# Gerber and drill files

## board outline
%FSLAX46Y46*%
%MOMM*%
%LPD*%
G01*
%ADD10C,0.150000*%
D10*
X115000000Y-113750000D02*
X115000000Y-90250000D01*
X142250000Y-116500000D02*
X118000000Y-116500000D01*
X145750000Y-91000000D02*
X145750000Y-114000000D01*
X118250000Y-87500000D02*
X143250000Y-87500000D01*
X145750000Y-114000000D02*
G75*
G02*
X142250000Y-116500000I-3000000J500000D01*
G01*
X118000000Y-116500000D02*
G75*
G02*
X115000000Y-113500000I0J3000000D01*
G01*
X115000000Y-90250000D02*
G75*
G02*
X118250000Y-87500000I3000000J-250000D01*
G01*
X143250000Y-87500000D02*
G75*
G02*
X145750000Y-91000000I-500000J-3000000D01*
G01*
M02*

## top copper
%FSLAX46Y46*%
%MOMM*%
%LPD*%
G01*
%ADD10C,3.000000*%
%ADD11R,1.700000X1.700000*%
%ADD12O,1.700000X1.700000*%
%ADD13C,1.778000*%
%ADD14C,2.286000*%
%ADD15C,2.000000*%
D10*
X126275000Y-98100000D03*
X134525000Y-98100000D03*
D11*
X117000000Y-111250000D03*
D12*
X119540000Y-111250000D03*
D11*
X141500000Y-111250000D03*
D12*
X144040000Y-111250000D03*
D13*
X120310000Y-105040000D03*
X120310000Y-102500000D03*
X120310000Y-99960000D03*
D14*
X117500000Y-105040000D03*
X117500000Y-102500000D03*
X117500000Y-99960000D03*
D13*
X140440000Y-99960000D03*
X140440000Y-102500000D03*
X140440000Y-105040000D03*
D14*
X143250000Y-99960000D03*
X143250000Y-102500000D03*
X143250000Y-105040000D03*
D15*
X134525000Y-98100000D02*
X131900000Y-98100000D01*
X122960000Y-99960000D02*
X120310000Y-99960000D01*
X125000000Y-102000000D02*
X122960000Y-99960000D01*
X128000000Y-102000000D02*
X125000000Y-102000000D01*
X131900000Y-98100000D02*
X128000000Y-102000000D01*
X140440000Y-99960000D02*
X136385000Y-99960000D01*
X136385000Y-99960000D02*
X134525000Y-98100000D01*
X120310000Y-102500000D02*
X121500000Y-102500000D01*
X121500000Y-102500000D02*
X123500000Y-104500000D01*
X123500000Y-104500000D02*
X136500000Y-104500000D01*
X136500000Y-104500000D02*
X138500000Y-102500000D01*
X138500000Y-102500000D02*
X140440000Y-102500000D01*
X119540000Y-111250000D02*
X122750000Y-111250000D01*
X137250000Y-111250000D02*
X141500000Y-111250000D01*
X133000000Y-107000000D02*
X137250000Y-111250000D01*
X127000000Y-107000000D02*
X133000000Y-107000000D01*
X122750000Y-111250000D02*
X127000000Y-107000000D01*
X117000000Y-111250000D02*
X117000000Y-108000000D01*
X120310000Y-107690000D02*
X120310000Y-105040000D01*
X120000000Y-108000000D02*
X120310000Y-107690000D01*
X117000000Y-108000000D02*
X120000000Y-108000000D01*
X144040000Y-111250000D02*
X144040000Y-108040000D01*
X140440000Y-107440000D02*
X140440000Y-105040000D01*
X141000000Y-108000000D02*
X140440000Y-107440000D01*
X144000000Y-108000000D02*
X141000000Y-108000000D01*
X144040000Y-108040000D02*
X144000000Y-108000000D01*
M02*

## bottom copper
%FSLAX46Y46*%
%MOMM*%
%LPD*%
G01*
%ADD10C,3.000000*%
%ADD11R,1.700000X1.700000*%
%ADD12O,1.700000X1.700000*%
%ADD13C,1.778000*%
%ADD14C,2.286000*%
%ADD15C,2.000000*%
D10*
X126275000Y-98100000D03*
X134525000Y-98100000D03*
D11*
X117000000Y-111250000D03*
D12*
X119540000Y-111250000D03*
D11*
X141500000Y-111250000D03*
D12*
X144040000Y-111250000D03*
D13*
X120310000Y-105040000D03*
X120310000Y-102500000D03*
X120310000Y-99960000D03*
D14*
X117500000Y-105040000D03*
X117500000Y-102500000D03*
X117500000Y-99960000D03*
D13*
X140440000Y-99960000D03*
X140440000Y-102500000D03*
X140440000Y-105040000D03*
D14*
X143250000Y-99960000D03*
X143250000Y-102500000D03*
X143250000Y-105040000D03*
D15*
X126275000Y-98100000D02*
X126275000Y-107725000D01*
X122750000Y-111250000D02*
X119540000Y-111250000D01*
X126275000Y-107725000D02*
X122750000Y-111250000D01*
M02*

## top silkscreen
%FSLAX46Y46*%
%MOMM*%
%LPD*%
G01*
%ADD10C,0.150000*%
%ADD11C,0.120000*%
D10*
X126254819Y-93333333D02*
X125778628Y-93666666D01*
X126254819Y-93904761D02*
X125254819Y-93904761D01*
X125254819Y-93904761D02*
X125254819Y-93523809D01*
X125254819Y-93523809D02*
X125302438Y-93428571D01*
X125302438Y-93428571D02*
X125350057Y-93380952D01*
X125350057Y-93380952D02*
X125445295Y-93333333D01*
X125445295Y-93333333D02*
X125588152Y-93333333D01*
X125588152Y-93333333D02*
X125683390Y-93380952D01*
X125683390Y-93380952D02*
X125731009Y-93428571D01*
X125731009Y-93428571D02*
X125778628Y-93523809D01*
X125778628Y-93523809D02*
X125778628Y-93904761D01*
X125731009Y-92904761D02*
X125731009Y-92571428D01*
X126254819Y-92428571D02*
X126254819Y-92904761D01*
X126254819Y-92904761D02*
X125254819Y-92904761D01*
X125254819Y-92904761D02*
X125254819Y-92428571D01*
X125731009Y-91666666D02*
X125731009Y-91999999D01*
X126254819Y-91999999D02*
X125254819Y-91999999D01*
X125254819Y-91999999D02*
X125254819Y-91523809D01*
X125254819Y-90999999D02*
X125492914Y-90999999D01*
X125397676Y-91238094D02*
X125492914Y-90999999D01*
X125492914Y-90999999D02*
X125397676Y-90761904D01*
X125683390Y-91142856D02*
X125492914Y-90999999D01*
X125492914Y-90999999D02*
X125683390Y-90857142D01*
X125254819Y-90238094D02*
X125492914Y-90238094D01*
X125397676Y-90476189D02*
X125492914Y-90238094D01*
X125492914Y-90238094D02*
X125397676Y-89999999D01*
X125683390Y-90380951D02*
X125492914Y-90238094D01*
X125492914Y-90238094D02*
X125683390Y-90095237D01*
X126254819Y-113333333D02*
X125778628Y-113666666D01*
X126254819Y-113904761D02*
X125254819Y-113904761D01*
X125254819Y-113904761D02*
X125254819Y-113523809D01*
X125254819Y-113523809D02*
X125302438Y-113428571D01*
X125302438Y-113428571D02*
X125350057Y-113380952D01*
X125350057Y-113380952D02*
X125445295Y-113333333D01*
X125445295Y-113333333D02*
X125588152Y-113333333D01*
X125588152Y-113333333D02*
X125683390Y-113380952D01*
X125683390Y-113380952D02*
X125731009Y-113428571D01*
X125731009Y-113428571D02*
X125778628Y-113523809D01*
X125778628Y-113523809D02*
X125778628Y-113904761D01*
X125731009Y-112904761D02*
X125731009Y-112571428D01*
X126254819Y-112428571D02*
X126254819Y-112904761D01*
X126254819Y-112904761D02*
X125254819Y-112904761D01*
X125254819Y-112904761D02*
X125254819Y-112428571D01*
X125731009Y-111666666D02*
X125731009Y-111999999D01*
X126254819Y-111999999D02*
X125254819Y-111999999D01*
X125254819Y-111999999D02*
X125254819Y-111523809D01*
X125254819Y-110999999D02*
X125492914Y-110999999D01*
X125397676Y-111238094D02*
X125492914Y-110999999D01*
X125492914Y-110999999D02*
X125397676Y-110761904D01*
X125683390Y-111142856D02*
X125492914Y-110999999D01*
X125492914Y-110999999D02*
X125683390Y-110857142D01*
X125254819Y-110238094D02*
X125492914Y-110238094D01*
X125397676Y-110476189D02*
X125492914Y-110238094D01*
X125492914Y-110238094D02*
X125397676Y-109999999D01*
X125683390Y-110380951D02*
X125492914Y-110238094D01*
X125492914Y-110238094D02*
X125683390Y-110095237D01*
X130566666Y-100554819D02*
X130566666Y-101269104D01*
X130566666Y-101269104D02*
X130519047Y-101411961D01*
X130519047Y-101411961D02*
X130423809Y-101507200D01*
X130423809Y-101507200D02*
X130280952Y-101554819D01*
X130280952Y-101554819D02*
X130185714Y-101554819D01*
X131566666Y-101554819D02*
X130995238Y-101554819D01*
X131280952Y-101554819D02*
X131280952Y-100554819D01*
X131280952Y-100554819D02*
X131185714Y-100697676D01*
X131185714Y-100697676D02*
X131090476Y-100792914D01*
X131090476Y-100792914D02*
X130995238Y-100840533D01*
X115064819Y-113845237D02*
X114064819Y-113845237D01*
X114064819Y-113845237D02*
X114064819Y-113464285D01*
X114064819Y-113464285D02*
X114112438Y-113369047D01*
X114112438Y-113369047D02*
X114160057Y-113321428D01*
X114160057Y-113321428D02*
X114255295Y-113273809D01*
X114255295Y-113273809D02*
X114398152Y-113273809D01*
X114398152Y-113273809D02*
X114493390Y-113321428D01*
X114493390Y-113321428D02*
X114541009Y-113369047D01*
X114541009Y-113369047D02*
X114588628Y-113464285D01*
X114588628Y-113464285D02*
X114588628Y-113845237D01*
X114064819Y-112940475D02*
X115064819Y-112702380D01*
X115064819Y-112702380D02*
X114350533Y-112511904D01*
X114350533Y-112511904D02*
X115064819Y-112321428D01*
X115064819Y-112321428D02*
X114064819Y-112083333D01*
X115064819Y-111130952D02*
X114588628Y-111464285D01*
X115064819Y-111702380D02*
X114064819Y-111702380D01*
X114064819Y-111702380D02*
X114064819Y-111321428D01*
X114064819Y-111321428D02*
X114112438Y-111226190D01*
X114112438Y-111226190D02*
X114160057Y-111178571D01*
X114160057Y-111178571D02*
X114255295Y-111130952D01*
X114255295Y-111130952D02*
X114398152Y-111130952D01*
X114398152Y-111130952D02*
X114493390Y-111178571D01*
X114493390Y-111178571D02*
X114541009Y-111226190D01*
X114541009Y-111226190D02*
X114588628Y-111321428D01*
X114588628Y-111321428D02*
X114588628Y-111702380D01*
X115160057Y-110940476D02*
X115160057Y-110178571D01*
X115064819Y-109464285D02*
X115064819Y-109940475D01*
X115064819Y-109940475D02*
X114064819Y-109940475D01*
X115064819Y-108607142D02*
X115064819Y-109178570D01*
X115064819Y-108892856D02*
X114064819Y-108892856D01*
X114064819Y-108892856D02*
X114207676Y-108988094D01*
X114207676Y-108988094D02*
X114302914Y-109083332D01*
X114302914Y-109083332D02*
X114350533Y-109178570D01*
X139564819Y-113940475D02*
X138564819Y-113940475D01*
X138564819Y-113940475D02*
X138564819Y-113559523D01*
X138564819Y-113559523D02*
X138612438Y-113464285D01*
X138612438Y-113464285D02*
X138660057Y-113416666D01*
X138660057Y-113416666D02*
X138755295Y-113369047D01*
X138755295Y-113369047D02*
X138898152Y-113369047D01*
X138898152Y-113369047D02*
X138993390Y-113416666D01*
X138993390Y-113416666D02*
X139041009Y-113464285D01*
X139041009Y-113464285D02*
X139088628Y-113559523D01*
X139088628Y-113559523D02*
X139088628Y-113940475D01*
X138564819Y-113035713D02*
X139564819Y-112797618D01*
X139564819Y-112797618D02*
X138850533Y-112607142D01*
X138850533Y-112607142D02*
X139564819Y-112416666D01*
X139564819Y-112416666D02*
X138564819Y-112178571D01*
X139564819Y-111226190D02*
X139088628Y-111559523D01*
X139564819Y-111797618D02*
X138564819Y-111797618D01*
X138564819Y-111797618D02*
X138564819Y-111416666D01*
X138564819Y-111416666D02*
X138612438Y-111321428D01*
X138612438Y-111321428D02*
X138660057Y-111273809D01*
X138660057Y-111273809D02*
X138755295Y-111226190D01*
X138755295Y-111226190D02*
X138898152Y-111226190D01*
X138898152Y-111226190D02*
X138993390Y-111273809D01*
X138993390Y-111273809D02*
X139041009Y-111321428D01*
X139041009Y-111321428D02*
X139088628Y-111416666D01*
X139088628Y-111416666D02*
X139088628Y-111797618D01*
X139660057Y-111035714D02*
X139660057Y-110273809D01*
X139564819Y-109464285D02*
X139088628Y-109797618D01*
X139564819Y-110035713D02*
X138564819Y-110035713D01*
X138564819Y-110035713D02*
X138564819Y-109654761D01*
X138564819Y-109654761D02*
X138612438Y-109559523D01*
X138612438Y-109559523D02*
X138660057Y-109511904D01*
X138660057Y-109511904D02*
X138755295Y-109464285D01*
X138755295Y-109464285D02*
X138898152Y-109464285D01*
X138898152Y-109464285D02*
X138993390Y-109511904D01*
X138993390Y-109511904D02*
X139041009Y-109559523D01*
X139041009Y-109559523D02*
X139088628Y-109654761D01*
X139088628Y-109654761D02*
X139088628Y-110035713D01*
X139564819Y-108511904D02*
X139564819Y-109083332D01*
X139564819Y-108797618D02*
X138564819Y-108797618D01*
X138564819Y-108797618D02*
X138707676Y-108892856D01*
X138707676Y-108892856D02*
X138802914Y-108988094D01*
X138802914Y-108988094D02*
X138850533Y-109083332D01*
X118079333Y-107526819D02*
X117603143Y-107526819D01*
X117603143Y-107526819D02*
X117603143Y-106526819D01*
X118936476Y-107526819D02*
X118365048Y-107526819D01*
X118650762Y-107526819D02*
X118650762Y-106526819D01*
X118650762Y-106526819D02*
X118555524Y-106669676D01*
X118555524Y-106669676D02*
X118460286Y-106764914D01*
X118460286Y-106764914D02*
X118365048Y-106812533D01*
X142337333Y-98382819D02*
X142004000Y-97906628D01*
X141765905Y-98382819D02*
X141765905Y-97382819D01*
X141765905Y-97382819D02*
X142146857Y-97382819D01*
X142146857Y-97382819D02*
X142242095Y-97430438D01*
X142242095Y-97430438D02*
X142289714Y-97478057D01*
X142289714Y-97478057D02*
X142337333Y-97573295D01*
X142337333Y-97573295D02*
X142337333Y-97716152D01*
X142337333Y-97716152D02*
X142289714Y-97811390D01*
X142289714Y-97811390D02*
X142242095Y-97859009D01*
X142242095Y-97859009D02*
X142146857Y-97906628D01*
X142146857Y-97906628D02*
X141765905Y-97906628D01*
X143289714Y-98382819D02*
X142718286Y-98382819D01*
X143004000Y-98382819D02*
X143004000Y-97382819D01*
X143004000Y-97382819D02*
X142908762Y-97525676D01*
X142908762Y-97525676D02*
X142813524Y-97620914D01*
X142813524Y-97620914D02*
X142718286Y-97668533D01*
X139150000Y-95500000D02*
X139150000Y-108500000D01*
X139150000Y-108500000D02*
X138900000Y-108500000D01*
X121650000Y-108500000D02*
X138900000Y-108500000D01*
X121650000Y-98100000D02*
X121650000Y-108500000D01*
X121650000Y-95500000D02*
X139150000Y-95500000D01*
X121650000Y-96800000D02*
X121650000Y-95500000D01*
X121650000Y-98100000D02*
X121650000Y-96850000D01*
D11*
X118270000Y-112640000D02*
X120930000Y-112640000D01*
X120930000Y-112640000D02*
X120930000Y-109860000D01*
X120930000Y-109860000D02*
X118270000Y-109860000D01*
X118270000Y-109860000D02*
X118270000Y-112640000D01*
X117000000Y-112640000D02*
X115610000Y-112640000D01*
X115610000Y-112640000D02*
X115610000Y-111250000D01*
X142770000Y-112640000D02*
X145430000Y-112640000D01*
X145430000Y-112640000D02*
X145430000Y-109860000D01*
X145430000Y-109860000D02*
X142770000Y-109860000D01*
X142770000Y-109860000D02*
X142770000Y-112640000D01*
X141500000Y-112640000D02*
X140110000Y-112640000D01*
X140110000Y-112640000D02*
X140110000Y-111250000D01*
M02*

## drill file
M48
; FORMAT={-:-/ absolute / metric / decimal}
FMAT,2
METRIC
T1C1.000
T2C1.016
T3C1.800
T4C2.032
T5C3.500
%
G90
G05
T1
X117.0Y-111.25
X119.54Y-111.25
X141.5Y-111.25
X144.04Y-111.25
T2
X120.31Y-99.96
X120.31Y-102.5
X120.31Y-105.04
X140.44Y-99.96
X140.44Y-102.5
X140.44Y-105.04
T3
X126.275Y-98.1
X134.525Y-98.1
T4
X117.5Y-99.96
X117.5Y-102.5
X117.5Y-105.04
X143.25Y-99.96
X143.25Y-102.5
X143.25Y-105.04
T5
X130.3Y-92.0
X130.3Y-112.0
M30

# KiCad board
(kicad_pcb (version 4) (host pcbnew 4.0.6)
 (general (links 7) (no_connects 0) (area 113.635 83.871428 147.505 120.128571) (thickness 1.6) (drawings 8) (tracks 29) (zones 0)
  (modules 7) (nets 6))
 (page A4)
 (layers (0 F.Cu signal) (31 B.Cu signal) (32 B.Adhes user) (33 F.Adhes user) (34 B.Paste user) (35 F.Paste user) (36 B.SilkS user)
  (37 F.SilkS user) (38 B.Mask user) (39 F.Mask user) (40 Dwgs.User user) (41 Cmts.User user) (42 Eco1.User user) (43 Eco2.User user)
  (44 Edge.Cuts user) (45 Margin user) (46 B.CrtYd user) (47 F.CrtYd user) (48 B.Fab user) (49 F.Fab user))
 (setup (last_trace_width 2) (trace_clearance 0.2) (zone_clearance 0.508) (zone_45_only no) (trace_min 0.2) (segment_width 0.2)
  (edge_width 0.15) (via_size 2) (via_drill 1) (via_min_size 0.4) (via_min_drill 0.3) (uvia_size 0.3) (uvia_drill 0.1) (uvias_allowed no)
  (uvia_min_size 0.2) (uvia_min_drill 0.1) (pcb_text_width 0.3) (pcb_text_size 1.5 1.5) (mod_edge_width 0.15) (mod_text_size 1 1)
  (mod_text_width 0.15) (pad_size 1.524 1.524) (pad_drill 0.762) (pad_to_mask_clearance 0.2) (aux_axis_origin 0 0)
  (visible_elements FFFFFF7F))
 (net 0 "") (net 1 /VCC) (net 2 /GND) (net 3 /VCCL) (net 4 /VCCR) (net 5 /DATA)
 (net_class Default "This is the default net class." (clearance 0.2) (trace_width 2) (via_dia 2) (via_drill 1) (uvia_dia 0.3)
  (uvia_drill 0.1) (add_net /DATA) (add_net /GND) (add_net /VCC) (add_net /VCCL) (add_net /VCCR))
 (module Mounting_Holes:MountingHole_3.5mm (layer F.Cu) (at 130.3 92 90)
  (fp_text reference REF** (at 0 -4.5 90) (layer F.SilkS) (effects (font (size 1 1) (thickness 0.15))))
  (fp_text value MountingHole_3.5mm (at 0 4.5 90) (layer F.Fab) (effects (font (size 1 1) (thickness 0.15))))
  (pad 1 np_thru_hole circle (at 0 0 90) (size 3.5 3.5) (drill 3.5) (layers *.Cu *.Mask)))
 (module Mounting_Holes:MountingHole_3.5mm (layer F.Cu) (at 130.3 112 90)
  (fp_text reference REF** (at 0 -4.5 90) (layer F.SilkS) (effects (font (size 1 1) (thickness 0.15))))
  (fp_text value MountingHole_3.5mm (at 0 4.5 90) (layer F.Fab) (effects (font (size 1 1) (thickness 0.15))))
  (pad 1 np_thru_hole circle (at 0 0 90) (size 3.5 3.5) (drill 3.5) (layers *.Cu *.Mask)))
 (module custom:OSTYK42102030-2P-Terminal (layer F.Cu) (at 130.4 98.1)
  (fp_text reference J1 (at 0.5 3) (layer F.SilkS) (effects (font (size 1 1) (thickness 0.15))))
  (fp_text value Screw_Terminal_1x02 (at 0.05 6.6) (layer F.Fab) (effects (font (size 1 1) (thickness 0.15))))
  (fp_line (start 8.75 -2.6) (end 8.75 10.4) (layer F.SilkS) (width 0.15))
  (fp_line (start 8.75 10.4) (end 8.5 10.4) (layer F.SilkS) (width 0.15))
  (fp_line (start -8.75 10.4) (end 8.5 10.4) (layer F.SilkS) (width 0.15))
  (fp_line (start -8.75 0) (end -8.75 10.4) (layer F.SilkS) (width 0.15))
  (fp_line (start -8.75 -2.6) (end 8.75 -2.6) (layer F.SilkS) (width 0.15))
  (fp_line (start -8.75 -1.3) (end -8.75 -2.6) (layer F.SilkS) (width 0.15))
  (fp_line (start -8.75 0) (end -8.75 -1.25) (layer F.SilkS) (width 0.15))
  (pad 1 thru_hole circle (at -4.125 0) (size 3 3) (drill 1.8) (layers *.Cu *.Mask) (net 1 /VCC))
  (pad 2 thru_hole circle (at 4.125 0) (size 3 3) (drill 1.8) (layers *.Cu *.Mask) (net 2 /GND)))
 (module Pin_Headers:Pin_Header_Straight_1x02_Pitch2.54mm (layer F.Cu) (at 117 111.25 90)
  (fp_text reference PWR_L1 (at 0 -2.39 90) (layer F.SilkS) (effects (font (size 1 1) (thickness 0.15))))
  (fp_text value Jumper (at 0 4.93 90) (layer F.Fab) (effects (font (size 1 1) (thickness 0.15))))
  (fp_line (start -1.39 1.27) (end -1.39 3.93) (layer F.SilkS) (width 0.12))
  (fp_line (start -1.39 3.93) (end 1.39 3.93) (layer F.SilkS) (width 0.12))
  (fp_line (start 1.39 3.93) (end 1.39 1.27) (layer F.SilkS) (width 0.12))
  (fp_line (start 1.39 1.27) (end -1.39 1.27) (layer F.SilkS) (width 0.12))
  (fp_line (start -1.39 0) (end -1.39 -1.39) (layer F.SilkS) (width 0.12))
  (fp_line (start -1.39 -1.39) (end 0 -1.39) (layer F.SilkS) (width 0.12))
  (pad 1 thru_hole rect (at 0 0 90) (size 1.7 1.7) (drill 1) (layers *.Cu *.Mask) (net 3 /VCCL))
  (pad 2 thru_hole oval (at 0 2.54 90) (size 1.7 1.7) (drill 1) (layers *.Cu *.Mask) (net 1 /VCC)))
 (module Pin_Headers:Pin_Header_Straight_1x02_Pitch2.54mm (layer F.Cu) (at 141.5 111.25 90)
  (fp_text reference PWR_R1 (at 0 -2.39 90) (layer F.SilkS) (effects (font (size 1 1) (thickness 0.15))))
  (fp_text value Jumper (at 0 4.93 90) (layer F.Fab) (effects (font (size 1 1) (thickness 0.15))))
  (fp_line (start -1.39 1.27) (end -1.39 3.93) (layer F.SilkS) (width 0.12))
  (fp_line (start -1.39 3.93) (end 1.39 3.93) (layer F.SilkS) (width 0.12))
  (fp_line (start 1.39 3.93) (end 1.39 1.27) (layer F.SilkS) (width 0.12))
  (fp_line (start 1.39 1.27) (end -1.39 1.27) (layer F.SilkS) (width 0.12))
  (fp_line (start -1.39 0) (end -1.39 -1.39) (layer F.SilkS) (width 0.12))
  (fp_line (start -1.39 -1.39) (end 0 -1.39) (layer F.SilkS) (width 0.12))
  (pad 1 thru_hole rect (at 0 0 90) (size 1.7 1.7) (drill 1) (layers *.Cu *.Mask) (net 1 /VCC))
  (pad 2 thru_hole oval (at 0 2.54 90) (size 1.7 1.7) (drill 1) (layers *.Cu *.Mask) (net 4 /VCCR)))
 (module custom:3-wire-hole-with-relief (layer F.Cu) (at 118.5 102.5 180)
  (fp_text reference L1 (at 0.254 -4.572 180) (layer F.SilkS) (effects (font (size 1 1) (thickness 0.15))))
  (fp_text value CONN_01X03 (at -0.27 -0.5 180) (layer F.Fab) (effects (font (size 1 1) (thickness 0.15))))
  (pad 1 thru_hole circle (at -1.81 -2.54 180) (size 1.778 1.778) (drill 1.016) (layers *.Cu *.Mask) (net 3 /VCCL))
  (pad 2 thru_hole circle (at -1.81 0 180) (size 1.778 1.778) (drill 1.016) (layers *.Cu *.Mask) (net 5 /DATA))
  (pad 3 thru_hole circle (at -1.81 2.54 180) (size 1.778 1.778) (drill 1.016) (layers *.Cu *.Mask) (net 2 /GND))
  (pad "" np_thru_hole circle (at 1 -2.54 180) (size 2.286 2.286) (drill 2.032) (layers *.Cu *.Mask))
  (pad "" np_thru_hole circle (at 1 0 180) (size 2.286 2.286) (drill 2.032) (layers *.Cu *.Mask))
  (pad "" np_thru_hole circle (at 1 2.54 180) (size 2.286 2.286) (drill 2.032) (layers *.Cu *.Mask)))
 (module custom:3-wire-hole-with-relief (layer F.Cu) (at 142.25 102.5)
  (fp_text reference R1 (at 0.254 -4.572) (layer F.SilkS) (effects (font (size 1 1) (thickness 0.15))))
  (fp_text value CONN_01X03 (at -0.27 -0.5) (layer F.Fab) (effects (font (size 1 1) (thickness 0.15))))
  (pad 1 thru_hole circle (at -1.81 -2.54) (size 1.778 1.778) (drill 1.016) (layers *.Cu *.Mask) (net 2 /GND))
  (pad 2 thru_hole circle (at -1.81 0) (size 1.778 1.778) (drill 1.016) (layers *.Cu *.Mask) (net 5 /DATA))
  (pad 3 thru_hole circle (at -1.81 2.54) (size 1.778 1.778) (drill 1.016) (layers *.Cu *.Mask) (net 4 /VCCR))
  (pad "" np_thru_hole circle (at 1 -2.54) (size 2.286 2.286) (drill 2.032) (layers *.Cu *.Mask))
  (pad "" np_thru_hole circle (at 1 0) (size 2.286 2.286) (drill 2.032) (layers *.Cu *.Mask))
  (pad "" np_thru_hole circle (at 1 2.54) (size 2.286 2.286) (drill 2.032) (layers *.Cu *.Mask)))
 (gr_line (start 115 113.75) (end 115 90.25) (angle 90) (layer Edge.Cuts) (width 0.15))
 (gr_line (start 142.25 116.5) (end 118 116.5) (angle 90) (layer Edge.Cuts) (width 0.15))
 (gr_line (start 145.75 91) (end 145.75 114) (angle 90) (layer Edge.Cuts) (width 0.15))
 (gr_line (start 118.25 87.5) (end 143.25 87.5) (angle 90) (layer Edge.Cuts) (width 0.15))
 (gr_arc (start 142.75 113.5) (end 145.75 114) (angle 90) (layer Edge.Cuts) (width 0.15))
 (gr_arc (start 118 113.5) (end 118 116.5) (angle 90) (layer Edge.Cuts) (width 0.15))
 (gr_arc (start 118 90.5) (end 115 90.25) (angle 90) (layer Edge.Cuts) (width 0.15))
 (gr_arc (start 142.75 90.5) (end 143.25 87.5) (angle 90) (layer Edge.Cuts) (width 0.15))
 (segment (start 134.525 98.1) (end 131.9 98.1) (width 2) (layer F.Cu) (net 2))
 (segment (start 122.96 99.96) (end 120.31 99.96) (width 2) (layer F.Cu) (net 2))
 (segment (start 125 102) (end 122.96 99.96) (width 2) (layer F.Cu) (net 2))
 (segment (start 128 102) (end 125 102) (width 2) (layer F.Cu) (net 2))
 (segment (start 131.9 98.1) (end 128 102) (width 2) (layer F.Cu) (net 2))
 (segment (start 140.44 99.96) (end 136.385 99.96) (width 2) (layer F.Cu) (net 2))
 (segment (start 136.385 99.96) (end 134.525 98.1) (width 2) (layer F.Cu) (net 2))
 (segment (start 120.31 102.5) (end 121.5 102.5) (width 2) (layer F.Cu) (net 5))
 (segment (start 121.5 102.5) (end 123.5 104.5) (width 2) (layer F.Cu) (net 5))
 (segment (start 123.5 104.5) (end 136.5 104.5) (width 2) (layer F.Cu) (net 5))
 (segment (start 136.5 104.5) (end 138.5 102.5) (width 2) (layer F.Cu) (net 5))
 (segment (start 138.5 102.5) (end 140.44 102.5) (width 2) (layer F.Cu) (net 5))
 (segment (start 126.275 98.1) (end 126.275 107.725) (width 2) (layer B.Cu) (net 1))
 (segment (start 122.75 111.25) (end 119.54 111.25) (width 2) (layer B.Cu) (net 1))
 (segment (start 126.275 107.725) (end 122.75 111.25) (width 2) (layer B.Cu) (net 1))
 (segment (start 119.54 111.25) (end 122.75 111.25) (width 2) (layer F.Cu) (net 1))
 (segment (start 137.25 111.25) (end 141.5 111.25) (width 2) (layer F.Cu) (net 1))
 (segment (start 133 107) (end 137.25 111.25) (width 2) (layer F.Cu) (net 1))
 (segment (start 127 107) (end 133 107) (width 2) (layer F.Cu) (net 1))
 (segment (start 122.75 111.25) (end 127 107) (width 2) (layer F.Cu) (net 1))
 (segment (start 117 111.25) (end 117 108) (width 2) (layer F.Cu) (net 3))
 (segment (start 120.31 107.69) (end 120.31 105.04) (width 2) (layer F.Cu) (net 3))
 (segment (start 120 108) (end 120.31 107.69) (width 2) (layer F.Cu) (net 3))
 (segment (start 117 108) (end 120 108) (width 2) (layer F.Cu) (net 3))
 (segment (start 144.04 111.25) (end 144.04 108.04) (width 2) (layer F.Cu) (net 4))
 (segment (start 140.44 107.44) (end 140.44 105.04) (width 2) (layer F.Cu) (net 4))
 (segment (start 141 108) (end 140.44 107.44) (width 2) (layer F.Cu) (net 4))
 (segment (start 144 108) (end 141 108) (width 2) (layer F.Cu) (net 4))
 (segment (start 144.04 108.04) (end 144 108) (width 2) (layer F.Cu) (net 4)))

